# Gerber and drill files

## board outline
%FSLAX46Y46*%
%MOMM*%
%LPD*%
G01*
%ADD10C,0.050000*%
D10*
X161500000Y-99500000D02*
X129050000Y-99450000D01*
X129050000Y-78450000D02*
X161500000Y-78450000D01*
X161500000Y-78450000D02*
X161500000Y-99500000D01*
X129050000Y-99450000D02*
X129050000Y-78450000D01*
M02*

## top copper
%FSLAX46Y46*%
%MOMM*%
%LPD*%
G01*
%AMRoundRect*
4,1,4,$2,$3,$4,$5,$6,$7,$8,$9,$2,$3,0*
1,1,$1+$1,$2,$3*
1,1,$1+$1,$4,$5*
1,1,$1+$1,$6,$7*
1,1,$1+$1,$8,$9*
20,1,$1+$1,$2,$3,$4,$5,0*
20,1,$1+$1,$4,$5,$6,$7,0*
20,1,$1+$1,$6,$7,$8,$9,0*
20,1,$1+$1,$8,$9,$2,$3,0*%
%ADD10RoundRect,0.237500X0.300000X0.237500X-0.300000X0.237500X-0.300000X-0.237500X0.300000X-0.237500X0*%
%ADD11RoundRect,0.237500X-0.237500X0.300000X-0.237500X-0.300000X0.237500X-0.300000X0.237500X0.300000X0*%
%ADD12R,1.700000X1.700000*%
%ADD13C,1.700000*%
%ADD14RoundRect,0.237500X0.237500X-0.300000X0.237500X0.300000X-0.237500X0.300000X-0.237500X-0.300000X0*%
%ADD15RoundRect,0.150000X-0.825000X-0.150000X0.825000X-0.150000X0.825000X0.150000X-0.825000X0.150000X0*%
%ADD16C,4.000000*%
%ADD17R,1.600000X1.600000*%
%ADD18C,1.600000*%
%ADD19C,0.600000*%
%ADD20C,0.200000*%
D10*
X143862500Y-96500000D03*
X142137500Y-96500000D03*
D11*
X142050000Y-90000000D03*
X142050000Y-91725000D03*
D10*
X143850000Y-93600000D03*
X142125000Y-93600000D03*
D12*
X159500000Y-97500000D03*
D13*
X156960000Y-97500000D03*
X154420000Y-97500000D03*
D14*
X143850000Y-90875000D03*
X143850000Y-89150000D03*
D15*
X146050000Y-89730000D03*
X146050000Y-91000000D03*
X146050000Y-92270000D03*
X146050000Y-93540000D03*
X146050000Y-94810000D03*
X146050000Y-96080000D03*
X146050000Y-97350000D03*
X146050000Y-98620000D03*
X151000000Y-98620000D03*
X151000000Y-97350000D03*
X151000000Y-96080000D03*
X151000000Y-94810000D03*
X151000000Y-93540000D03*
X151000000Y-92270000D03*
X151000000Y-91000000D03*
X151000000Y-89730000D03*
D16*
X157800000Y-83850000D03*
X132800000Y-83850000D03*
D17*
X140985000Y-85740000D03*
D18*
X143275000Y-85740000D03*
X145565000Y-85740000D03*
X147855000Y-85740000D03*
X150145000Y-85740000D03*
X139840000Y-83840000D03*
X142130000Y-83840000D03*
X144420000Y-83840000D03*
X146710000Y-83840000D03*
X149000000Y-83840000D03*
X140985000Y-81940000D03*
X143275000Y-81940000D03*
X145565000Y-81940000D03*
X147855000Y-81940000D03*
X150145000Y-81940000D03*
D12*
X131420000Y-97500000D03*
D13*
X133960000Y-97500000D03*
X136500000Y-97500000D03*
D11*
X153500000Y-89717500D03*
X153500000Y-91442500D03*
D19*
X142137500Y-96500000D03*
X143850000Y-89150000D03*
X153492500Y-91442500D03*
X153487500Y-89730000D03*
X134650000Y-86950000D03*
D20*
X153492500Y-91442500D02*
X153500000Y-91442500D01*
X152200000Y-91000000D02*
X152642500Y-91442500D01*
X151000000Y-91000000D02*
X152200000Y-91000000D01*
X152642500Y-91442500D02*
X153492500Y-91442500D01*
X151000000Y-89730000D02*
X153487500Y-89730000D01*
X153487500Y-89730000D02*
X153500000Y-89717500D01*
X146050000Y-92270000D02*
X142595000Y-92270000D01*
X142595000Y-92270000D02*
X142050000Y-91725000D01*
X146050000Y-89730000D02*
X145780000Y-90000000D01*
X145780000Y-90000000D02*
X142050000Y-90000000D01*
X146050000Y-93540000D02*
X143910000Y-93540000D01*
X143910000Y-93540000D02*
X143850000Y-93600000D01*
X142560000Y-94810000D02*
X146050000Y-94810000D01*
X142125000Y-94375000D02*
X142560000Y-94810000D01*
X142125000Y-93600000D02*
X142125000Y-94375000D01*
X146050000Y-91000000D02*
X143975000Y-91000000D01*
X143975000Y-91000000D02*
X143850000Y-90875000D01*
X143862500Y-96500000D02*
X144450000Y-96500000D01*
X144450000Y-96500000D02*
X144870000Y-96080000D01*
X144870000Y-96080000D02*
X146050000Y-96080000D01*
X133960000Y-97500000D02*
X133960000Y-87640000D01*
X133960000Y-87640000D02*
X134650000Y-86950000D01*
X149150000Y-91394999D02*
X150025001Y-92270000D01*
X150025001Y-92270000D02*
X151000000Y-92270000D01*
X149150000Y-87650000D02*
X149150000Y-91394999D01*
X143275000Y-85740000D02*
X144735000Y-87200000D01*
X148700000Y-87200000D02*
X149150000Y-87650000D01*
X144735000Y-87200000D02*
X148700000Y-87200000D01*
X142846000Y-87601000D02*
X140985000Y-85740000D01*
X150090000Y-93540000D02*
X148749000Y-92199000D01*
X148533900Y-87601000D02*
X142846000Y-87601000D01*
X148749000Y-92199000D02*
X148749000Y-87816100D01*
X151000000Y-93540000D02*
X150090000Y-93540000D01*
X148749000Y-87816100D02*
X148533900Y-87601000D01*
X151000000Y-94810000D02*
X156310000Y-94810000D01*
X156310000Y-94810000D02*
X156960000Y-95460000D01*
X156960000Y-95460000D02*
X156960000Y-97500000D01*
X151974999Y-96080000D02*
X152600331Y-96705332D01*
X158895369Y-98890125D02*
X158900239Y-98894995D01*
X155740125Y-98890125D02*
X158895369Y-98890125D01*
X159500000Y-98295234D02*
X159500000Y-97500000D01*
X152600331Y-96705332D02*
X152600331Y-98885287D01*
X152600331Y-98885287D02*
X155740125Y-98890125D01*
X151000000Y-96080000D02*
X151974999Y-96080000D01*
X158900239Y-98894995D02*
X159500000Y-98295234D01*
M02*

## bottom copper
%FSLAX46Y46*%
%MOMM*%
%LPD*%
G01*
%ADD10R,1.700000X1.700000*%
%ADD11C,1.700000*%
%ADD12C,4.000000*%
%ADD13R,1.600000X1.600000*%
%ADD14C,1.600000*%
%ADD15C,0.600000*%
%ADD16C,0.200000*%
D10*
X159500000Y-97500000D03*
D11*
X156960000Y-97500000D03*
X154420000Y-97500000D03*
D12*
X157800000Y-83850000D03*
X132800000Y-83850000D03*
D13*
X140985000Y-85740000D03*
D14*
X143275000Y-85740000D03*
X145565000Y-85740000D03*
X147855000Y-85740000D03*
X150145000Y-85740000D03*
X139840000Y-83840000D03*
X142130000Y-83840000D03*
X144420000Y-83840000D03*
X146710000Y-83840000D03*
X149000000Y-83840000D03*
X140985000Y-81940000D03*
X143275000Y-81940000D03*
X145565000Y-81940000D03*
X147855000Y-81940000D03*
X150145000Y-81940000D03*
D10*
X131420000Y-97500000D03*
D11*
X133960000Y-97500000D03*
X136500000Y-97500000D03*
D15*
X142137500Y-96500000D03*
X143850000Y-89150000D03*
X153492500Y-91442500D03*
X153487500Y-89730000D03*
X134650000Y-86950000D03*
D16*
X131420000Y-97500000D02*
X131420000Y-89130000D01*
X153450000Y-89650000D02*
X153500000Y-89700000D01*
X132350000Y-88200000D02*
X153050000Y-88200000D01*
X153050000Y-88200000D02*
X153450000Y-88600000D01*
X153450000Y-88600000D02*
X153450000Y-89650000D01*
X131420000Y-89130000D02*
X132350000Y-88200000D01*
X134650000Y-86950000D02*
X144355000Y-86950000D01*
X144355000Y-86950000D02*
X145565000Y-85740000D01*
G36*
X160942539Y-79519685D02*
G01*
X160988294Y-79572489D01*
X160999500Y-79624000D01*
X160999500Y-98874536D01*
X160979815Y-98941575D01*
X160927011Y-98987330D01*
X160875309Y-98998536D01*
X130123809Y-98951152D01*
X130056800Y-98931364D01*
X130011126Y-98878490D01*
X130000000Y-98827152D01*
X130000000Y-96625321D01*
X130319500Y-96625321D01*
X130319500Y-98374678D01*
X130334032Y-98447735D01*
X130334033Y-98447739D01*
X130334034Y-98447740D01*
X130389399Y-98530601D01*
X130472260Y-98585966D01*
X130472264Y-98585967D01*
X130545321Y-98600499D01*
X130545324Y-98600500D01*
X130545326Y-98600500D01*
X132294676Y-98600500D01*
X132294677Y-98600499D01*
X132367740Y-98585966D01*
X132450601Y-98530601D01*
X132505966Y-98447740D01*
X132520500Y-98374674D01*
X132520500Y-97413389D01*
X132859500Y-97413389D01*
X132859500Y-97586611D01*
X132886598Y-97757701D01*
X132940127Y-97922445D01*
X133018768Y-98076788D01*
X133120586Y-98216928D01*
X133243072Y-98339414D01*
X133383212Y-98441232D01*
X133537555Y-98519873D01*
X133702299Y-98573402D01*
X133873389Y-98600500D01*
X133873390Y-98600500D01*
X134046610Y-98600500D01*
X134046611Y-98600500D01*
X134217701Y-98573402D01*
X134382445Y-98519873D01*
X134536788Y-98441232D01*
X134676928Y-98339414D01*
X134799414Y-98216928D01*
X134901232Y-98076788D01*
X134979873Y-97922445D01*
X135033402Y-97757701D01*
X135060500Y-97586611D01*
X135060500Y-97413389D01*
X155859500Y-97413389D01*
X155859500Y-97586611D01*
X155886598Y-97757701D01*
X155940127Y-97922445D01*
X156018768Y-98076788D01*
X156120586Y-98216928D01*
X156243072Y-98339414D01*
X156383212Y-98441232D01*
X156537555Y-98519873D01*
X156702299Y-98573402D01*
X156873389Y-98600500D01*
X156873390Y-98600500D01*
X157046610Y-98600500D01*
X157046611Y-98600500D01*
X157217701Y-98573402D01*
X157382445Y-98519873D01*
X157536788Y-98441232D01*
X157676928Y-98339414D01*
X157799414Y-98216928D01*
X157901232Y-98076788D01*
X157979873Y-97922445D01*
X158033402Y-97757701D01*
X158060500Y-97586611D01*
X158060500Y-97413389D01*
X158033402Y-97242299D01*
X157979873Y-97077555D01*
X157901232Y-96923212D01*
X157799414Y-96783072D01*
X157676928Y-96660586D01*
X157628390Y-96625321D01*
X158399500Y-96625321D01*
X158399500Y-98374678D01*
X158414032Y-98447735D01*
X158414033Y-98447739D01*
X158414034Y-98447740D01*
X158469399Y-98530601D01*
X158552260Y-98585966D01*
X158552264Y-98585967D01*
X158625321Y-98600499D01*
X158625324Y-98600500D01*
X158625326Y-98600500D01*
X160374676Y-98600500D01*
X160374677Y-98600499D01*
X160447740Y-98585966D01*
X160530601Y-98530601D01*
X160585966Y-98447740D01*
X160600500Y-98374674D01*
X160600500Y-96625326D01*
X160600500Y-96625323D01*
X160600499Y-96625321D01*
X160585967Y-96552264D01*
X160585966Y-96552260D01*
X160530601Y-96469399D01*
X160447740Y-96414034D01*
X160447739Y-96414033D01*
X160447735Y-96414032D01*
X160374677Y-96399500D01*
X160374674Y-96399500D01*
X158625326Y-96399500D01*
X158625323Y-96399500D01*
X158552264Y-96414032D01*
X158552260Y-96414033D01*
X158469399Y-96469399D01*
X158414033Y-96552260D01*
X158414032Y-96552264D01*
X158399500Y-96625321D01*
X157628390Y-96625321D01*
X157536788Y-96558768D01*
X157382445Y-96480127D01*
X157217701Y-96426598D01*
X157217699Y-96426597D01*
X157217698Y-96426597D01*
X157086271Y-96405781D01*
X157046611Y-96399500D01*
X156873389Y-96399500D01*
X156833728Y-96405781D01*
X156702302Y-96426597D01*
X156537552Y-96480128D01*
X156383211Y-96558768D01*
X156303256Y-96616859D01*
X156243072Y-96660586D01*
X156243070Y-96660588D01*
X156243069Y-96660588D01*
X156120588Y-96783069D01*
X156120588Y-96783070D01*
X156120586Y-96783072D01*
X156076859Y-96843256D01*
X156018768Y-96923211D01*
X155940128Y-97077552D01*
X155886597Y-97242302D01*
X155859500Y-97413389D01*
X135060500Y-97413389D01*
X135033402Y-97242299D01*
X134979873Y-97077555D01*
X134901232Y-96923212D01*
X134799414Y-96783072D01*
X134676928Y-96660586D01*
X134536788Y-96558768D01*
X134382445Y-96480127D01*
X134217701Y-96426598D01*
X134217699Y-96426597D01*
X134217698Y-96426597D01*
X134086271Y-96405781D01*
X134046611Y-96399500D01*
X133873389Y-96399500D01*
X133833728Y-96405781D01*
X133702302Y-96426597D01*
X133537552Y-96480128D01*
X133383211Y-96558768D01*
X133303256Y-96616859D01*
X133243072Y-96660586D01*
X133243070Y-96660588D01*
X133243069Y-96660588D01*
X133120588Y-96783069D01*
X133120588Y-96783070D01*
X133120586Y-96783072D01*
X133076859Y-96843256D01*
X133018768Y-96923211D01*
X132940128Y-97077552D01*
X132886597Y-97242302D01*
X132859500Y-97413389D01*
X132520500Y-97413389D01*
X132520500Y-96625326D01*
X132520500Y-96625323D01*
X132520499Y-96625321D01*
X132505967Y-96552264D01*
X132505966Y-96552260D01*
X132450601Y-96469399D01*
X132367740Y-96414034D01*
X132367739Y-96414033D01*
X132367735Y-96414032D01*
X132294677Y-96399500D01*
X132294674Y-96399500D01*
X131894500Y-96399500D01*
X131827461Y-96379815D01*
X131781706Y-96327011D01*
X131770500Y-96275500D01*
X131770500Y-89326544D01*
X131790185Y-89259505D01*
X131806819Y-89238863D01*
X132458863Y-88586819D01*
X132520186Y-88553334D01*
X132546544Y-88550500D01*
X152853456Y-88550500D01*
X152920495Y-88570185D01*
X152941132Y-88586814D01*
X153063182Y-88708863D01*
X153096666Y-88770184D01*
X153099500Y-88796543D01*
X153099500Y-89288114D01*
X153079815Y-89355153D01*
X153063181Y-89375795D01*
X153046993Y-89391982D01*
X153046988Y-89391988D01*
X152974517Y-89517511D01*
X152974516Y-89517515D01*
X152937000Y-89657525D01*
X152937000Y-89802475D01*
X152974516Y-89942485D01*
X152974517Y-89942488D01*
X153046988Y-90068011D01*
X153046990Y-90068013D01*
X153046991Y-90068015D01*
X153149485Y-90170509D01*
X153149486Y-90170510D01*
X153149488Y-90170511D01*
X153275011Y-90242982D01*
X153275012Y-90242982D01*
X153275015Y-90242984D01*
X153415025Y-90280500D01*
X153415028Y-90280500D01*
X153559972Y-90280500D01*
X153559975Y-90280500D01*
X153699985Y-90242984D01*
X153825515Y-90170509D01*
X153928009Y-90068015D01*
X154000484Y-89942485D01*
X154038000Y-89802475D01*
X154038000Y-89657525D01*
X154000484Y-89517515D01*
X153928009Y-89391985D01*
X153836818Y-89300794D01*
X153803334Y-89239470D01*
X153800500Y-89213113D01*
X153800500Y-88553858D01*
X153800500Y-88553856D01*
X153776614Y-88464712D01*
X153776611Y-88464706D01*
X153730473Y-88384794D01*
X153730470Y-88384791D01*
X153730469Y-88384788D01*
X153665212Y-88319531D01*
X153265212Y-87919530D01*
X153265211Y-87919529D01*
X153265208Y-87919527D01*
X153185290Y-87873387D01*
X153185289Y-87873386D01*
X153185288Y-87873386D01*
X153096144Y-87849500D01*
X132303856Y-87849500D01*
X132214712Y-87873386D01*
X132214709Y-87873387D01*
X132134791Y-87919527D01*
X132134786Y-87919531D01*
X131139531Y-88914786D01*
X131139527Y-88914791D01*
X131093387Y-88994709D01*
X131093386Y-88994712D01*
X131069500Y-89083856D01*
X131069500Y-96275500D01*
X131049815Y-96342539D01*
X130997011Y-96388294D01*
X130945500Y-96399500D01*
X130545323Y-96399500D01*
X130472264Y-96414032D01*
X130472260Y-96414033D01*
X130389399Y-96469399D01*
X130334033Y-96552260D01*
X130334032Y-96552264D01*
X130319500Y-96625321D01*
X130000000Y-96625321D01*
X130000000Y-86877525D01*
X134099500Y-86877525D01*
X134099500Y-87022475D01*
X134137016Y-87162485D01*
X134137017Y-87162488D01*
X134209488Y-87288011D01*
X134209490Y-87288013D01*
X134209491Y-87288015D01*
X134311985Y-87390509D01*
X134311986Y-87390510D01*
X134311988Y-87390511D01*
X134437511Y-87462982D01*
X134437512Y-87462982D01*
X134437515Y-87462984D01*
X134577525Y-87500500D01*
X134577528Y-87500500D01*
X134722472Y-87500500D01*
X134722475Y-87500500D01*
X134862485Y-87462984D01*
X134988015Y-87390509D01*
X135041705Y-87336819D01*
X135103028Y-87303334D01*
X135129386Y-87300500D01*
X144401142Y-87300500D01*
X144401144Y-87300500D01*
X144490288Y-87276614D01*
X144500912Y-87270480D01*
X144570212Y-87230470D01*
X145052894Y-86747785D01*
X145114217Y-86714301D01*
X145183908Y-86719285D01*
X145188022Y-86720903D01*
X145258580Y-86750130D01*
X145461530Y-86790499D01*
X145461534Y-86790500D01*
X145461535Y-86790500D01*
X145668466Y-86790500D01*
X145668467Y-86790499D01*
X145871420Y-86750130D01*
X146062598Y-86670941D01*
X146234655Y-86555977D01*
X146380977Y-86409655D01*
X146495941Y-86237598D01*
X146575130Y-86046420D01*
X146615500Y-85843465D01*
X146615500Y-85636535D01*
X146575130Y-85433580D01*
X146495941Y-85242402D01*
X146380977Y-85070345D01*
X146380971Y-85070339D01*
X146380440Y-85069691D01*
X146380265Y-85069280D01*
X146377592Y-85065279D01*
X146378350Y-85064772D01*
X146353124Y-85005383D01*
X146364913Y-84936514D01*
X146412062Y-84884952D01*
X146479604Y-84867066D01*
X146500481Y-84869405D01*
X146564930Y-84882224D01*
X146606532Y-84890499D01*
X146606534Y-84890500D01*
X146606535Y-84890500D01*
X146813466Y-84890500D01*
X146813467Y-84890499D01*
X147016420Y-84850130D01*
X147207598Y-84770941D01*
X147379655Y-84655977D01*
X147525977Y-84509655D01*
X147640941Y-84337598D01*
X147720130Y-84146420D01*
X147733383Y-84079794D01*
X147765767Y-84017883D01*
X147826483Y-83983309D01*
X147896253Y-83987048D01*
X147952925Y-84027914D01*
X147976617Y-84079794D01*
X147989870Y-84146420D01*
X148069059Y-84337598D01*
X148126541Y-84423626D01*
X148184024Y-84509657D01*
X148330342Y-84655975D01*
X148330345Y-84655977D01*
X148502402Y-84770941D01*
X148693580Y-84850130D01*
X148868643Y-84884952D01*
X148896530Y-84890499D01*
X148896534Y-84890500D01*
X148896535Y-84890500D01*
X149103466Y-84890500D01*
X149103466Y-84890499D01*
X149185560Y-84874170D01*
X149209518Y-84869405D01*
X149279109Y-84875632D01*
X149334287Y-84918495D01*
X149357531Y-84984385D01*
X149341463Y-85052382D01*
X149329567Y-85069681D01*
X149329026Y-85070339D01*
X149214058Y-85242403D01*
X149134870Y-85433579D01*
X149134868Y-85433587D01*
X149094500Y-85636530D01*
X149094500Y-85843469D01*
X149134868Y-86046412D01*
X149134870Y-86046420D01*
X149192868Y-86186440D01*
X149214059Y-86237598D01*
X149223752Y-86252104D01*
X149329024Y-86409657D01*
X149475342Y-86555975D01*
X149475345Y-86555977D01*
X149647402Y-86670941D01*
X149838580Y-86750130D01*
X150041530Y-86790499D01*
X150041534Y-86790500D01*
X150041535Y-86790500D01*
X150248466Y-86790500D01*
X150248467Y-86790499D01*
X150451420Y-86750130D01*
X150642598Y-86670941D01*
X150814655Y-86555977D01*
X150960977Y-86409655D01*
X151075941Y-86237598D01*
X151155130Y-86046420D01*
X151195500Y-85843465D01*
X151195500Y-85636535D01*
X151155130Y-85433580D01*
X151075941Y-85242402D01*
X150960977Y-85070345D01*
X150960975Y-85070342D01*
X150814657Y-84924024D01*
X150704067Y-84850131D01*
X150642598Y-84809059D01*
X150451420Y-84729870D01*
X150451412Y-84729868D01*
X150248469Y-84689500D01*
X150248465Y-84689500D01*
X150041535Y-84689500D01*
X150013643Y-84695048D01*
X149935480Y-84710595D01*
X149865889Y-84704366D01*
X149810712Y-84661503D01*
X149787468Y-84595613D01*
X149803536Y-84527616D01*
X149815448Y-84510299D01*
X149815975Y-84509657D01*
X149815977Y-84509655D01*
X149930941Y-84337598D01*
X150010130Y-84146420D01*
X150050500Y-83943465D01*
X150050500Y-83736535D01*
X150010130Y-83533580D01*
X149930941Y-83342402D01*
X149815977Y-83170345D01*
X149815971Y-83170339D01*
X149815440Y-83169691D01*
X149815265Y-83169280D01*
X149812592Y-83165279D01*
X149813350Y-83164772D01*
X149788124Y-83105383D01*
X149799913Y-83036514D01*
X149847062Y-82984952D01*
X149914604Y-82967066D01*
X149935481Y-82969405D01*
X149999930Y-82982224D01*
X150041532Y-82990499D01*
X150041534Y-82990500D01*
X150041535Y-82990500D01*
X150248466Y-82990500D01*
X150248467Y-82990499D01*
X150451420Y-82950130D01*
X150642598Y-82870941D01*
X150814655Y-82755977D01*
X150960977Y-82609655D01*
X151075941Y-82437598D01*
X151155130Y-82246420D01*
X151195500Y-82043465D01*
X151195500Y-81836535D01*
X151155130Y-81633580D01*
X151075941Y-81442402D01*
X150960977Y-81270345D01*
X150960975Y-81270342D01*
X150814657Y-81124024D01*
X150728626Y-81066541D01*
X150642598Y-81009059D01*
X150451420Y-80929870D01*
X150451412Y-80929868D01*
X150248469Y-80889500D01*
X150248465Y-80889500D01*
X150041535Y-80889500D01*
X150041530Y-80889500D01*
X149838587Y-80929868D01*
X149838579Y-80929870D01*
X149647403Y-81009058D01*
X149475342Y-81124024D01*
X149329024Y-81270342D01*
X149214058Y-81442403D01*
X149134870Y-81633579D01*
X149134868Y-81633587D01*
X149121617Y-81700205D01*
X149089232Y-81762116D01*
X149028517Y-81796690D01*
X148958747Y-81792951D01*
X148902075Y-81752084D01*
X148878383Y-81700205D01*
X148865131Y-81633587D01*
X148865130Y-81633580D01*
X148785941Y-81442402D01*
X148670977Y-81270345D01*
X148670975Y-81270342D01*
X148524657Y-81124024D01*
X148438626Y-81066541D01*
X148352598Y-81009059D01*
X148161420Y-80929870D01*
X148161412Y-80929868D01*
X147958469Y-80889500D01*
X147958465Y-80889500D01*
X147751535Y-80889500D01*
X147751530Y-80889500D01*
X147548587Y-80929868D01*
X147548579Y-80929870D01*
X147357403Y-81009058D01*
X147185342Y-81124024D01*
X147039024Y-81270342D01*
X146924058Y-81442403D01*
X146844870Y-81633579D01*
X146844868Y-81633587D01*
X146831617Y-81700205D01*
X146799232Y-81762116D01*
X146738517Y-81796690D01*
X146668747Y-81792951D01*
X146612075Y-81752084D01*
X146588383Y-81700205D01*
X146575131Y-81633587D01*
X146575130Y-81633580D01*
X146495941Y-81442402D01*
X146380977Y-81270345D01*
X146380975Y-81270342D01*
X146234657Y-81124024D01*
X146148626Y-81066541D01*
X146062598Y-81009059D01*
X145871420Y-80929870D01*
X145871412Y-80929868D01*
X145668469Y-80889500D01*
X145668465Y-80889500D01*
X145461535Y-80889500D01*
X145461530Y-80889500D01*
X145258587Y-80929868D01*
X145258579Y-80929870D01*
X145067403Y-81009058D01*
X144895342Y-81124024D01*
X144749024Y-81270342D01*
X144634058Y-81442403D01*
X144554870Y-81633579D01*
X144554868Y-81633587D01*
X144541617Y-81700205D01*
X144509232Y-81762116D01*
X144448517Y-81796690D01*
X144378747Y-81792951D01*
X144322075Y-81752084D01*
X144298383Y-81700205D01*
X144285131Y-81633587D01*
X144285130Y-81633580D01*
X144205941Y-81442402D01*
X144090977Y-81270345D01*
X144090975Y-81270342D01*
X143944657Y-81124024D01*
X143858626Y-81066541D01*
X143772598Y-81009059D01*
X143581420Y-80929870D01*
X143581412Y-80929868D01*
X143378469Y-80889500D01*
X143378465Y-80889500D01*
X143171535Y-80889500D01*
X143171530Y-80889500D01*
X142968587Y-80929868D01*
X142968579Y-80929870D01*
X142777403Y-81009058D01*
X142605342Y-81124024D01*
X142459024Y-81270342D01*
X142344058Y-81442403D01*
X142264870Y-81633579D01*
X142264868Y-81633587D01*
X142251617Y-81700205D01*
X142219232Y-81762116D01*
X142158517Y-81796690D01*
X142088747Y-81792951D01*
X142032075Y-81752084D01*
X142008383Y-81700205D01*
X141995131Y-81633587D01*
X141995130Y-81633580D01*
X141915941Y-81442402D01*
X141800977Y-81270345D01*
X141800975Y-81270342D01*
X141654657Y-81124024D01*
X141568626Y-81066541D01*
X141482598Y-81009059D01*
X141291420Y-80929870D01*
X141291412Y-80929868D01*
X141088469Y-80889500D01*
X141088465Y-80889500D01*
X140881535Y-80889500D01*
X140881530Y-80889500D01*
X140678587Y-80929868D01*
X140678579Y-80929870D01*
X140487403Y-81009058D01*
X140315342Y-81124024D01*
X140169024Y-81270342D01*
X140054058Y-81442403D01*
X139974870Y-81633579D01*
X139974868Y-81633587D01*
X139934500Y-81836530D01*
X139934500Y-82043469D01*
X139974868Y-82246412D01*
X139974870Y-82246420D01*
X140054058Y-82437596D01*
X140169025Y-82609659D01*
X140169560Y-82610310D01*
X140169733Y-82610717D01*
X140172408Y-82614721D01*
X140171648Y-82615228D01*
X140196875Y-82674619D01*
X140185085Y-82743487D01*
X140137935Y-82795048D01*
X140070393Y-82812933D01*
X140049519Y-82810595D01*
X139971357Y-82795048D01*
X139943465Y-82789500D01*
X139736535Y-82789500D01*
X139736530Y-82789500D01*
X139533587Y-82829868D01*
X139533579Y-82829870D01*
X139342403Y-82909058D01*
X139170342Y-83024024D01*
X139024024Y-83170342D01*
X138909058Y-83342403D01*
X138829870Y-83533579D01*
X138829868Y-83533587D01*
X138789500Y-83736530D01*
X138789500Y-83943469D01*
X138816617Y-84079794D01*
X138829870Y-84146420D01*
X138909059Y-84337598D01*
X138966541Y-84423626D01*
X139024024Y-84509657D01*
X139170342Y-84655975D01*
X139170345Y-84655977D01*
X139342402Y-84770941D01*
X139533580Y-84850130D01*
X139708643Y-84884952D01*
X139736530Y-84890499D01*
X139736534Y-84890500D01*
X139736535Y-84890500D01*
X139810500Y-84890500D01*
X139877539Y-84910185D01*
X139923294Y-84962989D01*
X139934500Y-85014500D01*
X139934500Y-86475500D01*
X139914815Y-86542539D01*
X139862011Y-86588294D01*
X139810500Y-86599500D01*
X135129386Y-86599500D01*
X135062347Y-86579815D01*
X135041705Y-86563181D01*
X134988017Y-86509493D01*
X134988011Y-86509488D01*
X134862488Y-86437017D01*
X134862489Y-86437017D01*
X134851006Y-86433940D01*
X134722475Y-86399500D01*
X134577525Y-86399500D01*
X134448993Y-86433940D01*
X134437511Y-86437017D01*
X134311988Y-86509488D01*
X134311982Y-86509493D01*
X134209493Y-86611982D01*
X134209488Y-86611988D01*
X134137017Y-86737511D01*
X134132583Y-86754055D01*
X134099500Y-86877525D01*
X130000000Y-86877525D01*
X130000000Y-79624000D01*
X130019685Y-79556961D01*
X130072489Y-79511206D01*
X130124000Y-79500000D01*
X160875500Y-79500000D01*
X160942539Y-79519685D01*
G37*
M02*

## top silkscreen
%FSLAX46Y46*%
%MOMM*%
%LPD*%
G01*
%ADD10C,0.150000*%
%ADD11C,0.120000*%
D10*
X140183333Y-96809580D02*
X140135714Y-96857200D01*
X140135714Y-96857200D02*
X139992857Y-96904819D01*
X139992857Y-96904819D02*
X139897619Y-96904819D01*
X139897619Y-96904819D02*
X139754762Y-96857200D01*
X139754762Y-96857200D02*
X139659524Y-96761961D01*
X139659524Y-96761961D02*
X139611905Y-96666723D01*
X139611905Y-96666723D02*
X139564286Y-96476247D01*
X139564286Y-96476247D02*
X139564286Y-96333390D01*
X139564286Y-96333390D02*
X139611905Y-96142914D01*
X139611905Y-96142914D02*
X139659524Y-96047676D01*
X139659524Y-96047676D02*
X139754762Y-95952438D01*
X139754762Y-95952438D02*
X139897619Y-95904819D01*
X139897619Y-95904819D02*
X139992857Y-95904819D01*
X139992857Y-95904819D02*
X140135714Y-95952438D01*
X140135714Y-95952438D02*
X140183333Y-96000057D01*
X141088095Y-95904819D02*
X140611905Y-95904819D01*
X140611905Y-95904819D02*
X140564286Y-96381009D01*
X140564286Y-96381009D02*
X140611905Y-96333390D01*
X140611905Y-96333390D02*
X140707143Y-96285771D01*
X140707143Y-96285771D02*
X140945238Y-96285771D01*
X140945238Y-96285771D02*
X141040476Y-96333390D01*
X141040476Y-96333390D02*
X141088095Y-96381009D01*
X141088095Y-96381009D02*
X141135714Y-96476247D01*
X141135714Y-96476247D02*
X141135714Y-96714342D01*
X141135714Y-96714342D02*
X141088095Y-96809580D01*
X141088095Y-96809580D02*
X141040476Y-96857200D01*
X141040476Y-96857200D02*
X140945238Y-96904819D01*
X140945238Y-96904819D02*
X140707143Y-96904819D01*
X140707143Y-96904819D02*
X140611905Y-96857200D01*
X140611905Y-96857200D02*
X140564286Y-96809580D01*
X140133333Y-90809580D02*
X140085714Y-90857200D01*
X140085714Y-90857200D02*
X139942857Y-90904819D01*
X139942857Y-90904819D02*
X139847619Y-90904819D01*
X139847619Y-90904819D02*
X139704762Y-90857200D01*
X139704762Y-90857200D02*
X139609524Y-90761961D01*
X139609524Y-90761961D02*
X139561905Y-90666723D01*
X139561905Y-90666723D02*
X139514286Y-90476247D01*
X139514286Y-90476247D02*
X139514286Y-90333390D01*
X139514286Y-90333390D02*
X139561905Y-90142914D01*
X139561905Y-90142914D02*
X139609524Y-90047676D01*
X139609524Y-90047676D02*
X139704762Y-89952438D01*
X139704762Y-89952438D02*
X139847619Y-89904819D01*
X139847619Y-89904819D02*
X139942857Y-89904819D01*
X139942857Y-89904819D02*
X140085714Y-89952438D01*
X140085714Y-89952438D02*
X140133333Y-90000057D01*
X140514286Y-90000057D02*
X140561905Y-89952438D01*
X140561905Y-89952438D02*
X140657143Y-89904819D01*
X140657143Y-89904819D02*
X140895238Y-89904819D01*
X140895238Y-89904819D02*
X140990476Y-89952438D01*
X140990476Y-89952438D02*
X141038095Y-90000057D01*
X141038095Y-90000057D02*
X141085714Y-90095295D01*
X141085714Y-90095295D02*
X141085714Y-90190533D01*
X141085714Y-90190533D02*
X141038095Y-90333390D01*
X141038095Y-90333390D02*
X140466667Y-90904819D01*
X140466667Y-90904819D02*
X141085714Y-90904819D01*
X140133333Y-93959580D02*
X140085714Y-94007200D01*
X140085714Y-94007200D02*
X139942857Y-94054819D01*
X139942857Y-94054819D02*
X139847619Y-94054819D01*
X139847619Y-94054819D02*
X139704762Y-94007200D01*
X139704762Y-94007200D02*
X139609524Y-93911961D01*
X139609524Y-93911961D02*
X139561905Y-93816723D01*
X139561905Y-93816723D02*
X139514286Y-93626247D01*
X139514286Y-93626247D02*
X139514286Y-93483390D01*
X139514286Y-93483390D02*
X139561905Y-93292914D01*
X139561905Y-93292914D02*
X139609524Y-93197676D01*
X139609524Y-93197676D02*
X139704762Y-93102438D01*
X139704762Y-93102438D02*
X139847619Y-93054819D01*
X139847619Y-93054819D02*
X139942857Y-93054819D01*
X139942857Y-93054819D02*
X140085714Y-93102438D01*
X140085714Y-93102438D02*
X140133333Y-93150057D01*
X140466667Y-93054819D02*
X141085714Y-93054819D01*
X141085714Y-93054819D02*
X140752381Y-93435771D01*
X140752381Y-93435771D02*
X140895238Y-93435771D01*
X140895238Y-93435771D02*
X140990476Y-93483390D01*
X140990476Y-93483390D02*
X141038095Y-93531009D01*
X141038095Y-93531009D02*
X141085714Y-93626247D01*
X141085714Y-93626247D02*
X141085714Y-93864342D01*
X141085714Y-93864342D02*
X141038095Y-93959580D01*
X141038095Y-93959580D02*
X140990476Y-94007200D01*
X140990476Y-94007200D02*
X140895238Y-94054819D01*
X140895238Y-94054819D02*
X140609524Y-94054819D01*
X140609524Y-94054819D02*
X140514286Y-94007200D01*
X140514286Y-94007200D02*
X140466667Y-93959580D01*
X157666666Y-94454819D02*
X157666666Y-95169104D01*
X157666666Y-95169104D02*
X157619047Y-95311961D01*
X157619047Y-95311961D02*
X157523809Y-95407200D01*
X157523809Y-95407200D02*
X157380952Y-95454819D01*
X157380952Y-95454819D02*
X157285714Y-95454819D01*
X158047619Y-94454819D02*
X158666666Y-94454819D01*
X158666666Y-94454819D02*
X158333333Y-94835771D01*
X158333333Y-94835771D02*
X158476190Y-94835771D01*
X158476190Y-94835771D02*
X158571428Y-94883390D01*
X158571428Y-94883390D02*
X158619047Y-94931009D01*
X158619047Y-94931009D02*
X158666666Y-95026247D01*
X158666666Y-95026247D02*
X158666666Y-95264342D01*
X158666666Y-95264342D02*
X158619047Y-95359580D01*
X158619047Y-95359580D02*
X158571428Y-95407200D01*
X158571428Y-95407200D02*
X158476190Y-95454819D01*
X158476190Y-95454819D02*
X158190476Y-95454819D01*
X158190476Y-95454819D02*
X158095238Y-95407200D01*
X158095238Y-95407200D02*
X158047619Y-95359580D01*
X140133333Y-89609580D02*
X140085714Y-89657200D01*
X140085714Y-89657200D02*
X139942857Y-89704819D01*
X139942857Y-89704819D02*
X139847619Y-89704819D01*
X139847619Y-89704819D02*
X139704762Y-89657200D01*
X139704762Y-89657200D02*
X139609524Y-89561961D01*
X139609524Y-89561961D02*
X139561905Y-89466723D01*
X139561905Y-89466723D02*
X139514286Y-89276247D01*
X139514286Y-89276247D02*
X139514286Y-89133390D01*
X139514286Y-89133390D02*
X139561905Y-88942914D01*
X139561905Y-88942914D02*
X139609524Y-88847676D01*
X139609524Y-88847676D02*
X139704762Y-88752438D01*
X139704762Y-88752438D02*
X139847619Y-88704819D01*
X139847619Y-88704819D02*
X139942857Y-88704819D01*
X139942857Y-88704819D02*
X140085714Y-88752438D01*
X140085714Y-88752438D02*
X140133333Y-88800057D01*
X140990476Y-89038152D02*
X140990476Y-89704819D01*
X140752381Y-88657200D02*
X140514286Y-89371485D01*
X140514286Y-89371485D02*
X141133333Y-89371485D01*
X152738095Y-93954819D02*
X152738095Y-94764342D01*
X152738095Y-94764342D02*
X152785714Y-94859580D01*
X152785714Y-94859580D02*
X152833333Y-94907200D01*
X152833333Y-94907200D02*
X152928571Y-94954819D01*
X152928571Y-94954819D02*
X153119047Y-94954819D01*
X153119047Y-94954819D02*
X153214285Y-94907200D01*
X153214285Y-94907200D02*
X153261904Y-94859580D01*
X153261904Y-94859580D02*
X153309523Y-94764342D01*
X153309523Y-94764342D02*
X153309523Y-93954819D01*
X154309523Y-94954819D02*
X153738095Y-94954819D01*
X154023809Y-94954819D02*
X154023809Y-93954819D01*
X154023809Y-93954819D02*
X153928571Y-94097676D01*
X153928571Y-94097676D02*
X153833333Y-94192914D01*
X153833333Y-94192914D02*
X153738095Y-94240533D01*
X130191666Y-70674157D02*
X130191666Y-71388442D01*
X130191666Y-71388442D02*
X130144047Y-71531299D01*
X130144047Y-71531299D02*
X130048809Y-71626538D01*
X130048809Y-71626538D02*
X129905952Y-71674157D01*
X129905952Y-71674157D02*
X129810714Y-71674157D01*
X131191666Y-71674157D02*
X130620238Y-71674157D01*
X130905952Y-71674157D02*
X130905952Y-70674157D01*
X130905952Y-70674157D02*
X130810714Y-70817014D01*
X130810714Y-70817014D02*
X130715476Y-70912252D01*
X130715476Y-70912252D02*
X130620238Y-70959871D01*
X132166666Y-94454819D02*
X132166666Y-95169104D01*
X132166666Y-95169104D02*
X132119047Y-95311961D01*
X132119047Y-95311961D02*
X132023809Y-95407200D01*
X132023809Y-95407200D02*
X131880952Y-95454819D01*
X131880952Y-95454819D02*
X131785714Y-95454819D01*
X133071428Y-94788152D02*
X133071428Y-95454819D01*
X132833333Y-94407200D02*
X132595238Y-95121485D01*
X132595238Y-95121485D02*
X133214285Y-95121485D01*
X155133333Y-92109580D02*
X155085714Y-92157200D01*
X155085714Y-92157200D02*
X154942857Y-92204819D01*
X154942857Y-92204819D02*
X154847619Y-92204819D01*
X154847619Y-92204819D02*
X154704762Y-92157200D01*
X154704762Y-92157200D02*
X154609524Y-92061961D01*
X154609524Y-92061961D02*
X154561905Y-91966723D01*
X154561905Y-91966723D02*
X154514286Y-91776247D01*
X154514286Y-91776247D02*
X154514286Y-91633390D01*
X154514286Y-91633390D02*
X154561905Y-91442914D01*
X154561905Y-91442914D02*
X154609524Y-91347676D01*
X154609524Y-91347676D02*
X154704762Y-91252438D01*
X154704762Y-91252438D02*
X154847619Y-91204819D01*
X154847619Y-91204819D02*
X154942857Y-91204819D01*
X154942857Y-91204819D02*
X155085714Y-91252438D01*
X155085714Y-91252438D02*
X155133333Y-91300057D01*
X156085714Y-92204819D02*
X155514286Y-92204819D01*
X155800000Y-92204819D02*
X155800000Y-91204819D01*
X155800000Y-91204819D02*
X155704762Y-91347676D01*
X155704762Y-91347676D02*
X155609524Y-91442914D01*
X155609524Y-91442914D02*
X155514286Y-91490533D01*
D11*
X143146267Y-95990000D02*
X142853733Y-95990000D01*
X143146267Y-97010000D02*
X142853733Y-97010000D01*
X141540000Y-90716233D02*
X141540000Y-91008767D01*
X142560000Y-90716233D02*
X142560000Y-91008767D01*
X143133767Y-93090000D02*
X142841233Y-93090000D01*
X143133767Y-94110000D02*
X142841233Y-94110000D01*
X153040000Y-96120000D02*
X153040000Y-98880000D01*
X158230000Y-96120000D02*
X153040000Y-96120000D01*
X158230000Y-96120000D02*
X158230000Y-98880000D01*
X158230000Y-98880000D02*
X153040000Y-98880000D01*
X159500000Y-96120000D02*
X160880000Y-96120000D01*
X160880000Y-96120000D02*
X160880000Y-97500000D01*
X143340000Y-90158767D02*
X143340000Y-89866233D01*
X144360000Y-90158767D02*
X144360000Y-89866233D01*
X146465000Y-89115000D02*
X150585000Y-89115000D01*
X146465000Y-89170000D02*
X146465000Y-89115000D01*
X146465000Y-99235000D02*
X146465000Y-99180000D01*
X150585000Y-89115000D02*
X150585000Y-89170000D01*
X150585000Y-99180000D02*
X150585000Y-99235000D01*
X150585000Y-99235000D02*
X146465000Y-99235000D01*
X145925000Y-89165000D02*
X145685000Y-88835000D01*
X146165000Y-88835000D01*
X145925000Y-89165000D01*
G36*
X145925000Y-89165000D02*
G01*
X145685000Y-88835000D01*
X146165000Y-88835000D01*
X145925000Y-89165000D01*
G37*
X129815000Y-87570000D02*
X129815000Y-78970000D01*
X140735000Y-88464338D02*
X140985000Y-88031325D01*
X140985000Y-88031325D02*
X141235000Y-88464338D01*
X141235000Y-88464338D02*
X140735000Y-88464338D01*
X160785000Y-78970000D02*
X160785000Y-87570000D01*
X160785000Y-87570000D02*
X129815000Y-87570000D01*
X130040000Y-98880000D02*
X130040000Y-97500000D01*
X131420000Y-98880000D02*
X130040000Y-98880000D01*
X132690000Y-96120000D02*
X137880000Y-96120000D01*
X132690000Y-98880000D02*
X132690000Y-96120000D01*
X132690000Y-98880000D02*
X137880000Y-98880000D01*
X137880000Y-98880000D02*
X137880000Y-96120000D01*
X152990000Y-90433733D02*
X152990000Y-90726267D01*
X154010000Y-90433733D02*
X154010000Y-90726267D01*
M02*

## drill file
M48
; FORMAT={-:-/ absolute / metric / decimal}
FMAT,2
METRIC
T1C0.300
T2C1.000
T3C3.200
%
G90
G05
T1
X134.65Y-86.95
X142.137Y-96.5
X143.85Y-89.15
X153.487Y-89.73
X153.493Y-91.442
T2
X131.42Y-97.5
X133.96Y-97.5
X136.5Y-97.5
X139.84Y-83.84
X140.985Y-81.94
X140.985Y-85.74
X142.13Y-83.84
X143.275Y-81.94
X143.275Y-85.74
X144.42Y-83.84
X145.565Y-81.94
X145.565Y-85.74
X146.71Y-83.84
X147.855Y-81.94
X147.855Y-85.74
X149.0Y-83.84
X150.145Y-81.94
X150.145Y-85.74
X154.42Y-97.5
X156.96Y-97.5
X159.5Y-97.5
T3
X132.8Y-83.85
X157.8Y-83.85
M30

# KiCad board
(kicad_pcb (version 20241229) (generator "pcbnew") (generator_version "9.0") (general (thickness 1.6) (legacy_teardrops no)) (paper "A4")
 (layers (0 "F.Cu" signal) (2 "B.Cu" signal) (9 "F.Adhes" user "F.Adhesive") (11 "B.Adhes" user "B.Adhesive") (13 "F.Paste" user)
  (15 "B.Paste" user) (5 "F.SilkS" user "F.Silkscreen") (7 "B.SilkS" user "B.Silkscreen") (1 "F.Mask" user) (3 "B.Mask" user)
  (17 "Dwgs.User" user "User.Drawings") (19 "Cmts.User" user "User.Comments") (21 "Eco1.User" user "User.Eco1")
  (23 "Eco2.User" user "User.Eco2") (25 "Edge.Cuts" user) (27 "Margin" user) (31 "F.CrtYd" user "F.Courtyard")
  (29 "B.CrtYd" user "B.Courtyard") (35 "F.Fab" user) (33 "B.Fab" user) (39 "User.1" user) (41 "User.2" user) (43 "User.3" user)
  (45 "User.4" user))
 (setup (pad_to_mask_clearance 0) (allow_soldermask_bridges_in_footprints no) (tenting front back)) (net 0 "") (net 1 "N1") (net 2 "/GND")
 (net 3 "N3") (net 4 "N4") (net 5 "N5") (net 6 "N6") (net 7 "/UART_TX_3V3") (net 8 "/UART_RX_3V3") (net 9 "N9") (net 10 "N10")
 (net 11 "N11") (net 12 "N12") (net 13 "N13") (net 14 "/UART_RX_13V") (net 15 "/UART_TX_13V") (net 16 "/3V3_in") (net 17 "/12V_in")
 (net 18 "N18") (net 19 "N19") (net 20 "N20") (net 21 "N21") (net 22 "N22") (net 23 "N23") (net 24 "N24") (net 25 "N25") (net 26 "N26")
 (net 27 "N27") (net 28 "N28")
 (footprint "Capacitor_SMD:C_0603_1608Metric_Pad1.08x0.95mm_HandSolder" (layer "F.Cu") (at 143 96.5 180)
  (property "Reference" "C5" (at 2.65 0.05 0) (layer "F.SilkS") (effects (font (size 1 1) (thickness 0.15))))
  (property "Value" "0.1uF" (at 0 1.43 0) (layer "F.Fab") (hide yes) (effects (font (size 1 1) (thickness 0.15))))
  (fp_line (start -0.146267 0.51) (end 0.146267 0.51) (stroke (width 0.12) (type solid)) (layer "F.SilkS"))
  (fp_line (start -0.146267 -0.51) (end 0.146267 -0.51) (stroke (width 0.12) (type solid)) (layer "F.SilkS"))
  (pad "1" smd roundrect (at -0.8625 0 180) (size 1.075 0.95) (layers "F.Cu" "F.Mask" "F.Paste") (roundrect_rratio 0.25) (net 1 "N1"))
  (pad "2" smd roundrect (at 0.8625 0 180) (size 1.075 0.95) (layers "F.Cu" "F.Mask" "F.Paste") (roundrect_rratio 0.25) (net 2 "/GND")))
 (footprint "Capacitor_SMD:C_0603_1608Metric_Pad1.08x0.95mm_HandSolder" (layer "F.Cu") (at 142.05 90.8625 -90)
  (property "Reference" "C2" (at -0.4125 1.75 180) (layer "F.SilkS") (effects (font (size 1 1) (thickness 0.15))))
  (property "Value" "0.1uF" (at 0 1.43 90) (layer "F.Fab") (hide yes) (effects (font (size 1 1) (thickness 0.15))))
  (fp_line (start -0.146267 0.51) (end 0.146267 0.51) (stroke (width 0.12) (type solid)) (layer "F.SilkS"))
  (fp_line (start -0.146267 -0.51) (end 0.146267 -0.51) (stroke (width 0.12) (type solid)) (layer "F.SilkS"))
  (pad "1" smd roundrect (at -0.8625 0 270) (size 1.075 0.95) (layers "F.Cu" "F.Mask" "F.Paste") (roundrect_rratio 0.25) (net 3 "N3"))
  (pad "2" smd roundrect (at 0.8625 0 270) (size 1.075 0.95) (layers "F.Cu" "F.Mask" "F.Paste") (roundrect_rratio 0.25) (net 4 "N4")))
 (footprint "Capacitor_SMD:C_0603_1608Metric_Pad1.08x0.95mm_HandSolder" (layer "F.Cu") (at 142.9875 93.6 180)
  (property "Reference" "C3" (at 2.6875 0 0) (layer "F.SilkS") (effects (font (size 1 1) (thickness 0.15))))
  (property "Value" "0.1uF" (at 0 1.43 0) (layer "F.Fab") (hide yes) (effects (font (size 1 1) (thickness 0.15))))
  (fp_line (start -0.146267 0.51) (end 0.146267 0.51) (stroke (width 0.12) (type solid)) (layer "F.SilkS"))
  (fp_line (start -0.146267 -0.51) (end 0.146267 -0.51) (stroke (width 0.12) (type solid)) (layer "F.SilkS"))
  (pad "1" smd roundrect (at -0.8625 0 180) (size 1.075 0.95) (layers "F.Cu" "F.Mask" "F.Paste") (roundrect_rratio 0.25) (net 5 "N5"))
  (pad "2" smd roundrect (at 0.8625 0 180) (size 1.075 0.95) (layers "F.Cu" "F.Mask" "F.Paste") (roundrect_rratio 0.25) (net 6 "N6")))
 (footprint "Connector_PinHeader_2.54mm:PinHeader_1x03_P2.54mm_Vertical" (layer "F.Cu") (at 159.5 97.5 -90)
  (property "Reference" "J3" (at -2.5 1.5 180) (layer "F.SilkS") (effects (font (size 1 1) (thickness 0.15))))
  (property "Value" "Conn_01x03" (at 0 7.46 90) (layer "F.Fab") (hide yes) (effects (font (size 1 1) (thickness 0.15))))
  (fp_line (start -1.38 6.46) (end 1.38 6.46) (stroke (width 0.12) (type solid)) (layer "F.SilkS"))
  (fp_line (start -1.38 1.27) (end -1.38 6.46) (stroke (width 0.12) (type solid)) (layer "F.SilkS"))
  (fp_line (start -1.38 1.27) (end 1.38 1.27) (stroke (width 0.12) (type solid)) (layer "F.SilkS"))
  (fp_line (start 1.38 1.27) (end 1.38 6.46) (stroke (width 0.12) (type solid)) (layer "F.SilkS"))
  (fp_line (start -1.38 0) (end -1.38 -1.38) (stroke (width 0.12) (type solid)) (layer "F.SilkS"))
  (fp_line (start -1.38 -1.38) (end 0 -1.38) (stroke (width 0.12) (type solid)) (layer "F.SilkS"))
  (pad "1" thru_hole rect (at 0 0 270) (size 1.7 1.7) (drill 1) (layers "*.Cu" "*.Mask") (remove_unused_layers no) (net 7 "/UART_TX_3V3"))
  (pad "2" thru_hole circle (at 0 2.54 270) (size 1.7 1.7) (drill 1) (layers "*.Cu" "*.Mask") (remove_unused_layers no)
   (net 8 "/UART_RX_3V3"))
  (pad "3" thru_hole circle (at 0 5.08 270) (size 1.7 1.7) (drill 1) (layers "*.Cu" "*.Mask") (remove_unused_layers no) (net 2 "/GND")))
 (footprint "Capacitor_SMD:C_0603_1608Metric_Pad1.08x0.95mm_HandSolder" (layer "F.Cu") (at 143.85 90.0125 90)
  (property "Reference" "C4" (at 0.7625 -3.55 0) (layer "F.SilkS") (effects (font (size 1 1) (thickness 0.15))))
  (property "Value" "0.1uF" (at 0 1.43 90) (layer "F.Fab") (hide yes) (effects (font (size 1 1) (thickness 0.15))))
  (fp_line (start -0.146267 -0.51) (end 0.146267 -0.51) (stroke (width 0.12) (type solid)) (layer "F.SilkS"))
  (fp_line (start -0.146267 0.51) (end 0.146267 0.51) (stroke (width 0.12) (type solid)) (layer "F.SilkS"))
  (pad "1" smd roundrect (at -0.8625 0 90) (size 1.075 0.95) (layers "F.Cu" "F.Mask" "F.Paste") (roundrect_rratio 0.25) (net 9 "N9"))
  (pad "2" smd roundrect (at 0.8625 0 90) (size 1.075 0.95) (layers "F.Cu" "F.Mask" "F.Paste") (roundrect_rratio 0.25) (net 2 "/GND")))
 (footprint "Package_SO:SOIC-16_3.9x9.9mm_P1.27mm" (layer "F.Cu") (at 148.525 94.175)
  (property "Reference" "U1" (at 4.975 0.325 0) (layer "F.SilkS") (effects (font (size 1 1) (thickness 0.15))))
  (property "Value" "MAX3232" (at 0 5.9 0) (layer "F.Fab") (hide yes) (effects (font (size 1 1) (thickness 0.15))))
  (fp_line (start -2.06 -5.06) (end 2.06 -5.06) (stroke (width 0.12) (type solid)) (layer "F.SilkS"))
  (fp_line (start -2.06 -5.005) (end -2.06 -5.06) (stroke (width 0.12) (type solid)) (layer "F.SilkS"))
  (fp_line (start -2.06 5.06) (end -2.06 5.005) (stroke (width 0.12) (type solid)) (layer "F.SilkS"))
  (fp_line (start 2.06 -5.06) (end 2.06 -5.005) (stroke (width 0.12) (type solid)) (layer "F.SilkS"))
  (fp_line (start 2.06 5.005) (end 2.06 5.06) (stroke (width 0.12) (type solid)) (layer "F.SilkS"))
  (fp_line (start 2.06 5.06) (end -2.06 5.06) (stroke (width 0.12) (type solid)) (layer "F.SilkS"))
  (fp_poly (pts (xy -2.6 -5.01) (xy -2.84 -5.34) (xy -2.36 -5.34)) (stroke (width 0.12) (type solid)) (fill yes) (layer "F.SilkS"))
  (pad "1" smd roundrect (at -2.475 -4.445) (size 1.95 0.6) (layers "F.Cu" "F.Mask" "F.Paste") (roundrect_rratio 0.25) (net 3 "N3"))
  (pad "2" smd roundrect (at -2.475 -3.175) (size 1.95 0.6) (layers "F.Cu" "F.Mask" "F.Paste") (roundrect_rratio 0.25) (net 9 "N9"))
  (pad "3" smd roundrect (at -2.475 -1.905) (size 1.95 0.6) (layers "F.Cu" "F.Mask" "F.Paste") (roundrect_rratio 0.25) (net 4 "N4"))
  (pad "4" smd roundrect (at -2.475 -0.635) (size 1.95 0.6) (layers "F.Cu" "F.Mask" "F.Paste") (roundrect_rratio 0.25) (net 5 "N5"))
  (pad "5" smd roundrect (at -2.475 0.635) (size 1.95 0.6) (layers "F.Cu" "F.Mask" "F.Paste") (roundrect_rratio 0.25) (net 6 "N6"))
  (pad "6" smd roundrect (at -2.475 1.905) (size 1.95 0.6) (layers "F.Cu" "F.Mask" "F.Paste") (roundrect_rratio 0.25) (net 1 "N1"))
  (pad "7" smd roundrect (at -2.475 3.175) (size 1.95 0.6) (layers "F.Cu" "F.Mask" "F.Paste") (roundrect_rratio 0.25) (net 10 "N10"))
  (pad "8" smd roundrect (at -2.475 4.445) (size 1.95 0.6) (layers "F.Cu" "F.Mask" "F.Paste") (roundrect_rratio 0.25) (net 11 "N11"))
  (pad "9" smd roundrect (at 2.475 4.445) (size 1.95 0.6) (layers "F.Cu" "F.Mask" "F.Paste") (roundrect_rratio 0.25) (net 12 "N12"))
  (pad "10" smd roundrect (at 2.475 3.175) (size 1.95 0.6) (layers "F.Cu" "F.Mask" "F.Paste") (roundrect_rratio 0.25) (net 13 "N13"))
  (pad "11" smd roundrect (at 2.475 1.905) (size 1.95 0.6) (layers "F.Cu" "F.Mask" "F.Paste") (roundrect_rratio 0.25) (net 7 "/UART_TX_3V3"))
  (pad "12" smd roundrect (at 2.475 0.635) (size 1.95 0.6) (layers "F.Cu" "F.Mask" "F.Paste") (roundrect_rratio 0.25) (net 8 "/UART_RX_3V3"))
  (pad "13" smd roundrect (at 2.475 -0.635) (size 1.95 0.6) (layers "F.Cu" "F.Mask" "F.Paste") (roundrect_rratio 0.25)
   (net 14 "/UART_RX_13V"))
  (pad "14" smd roundrect (at 2.475 -1.905) (size 1.95 0.6) (layers "F.Cu" "F.Mask" "F.Paste") (roundrect_rratio 0.25)
   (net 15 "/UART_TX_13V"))
  (pad "15" smd roundrect (at 2.475 -3.175) (size 1.95 0.6) (layers "F.Cu" "F.Mask" "F.Paste") (roundrect_rratio 0.25) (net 2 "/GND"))
  (pad "16" smd roundrect (at 2.475 -4.445) (size 1.95 0.6) (layers "F.Cu" "F.Mask" "F.Paste") (roundrect_rratio 0.25) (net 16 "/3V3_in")))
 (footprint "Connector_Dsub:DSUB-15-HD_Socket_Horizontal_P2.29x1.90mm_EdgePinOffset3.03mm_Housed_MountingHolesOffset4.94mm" (layer "F.Cu")
  (at 140.985 85.74 180)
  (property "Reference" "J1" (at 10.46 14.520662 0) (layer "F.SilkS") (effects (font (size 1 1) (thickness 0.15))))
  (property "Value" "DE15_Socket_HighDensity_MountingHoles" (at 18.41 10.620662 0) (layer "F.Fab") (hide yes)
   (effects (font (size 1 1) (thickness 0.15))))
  (fp_line (start 11.17 -1.83) (end 11.17 6.77) (stroke (width 0.12) (type solid)) (layer "F.SilkS"))
  (fp_line (start 0.25 -2.724338) (end 0 -2.291325) (stroke (width 0.12) (type solid)) (layer "F.SilkS"))
  (fp_line (start 0 -2.291325) (end -0.25 -2.724338) (stroke (width 0.12) (type solid)) (layer "F.SilkS"))
  (fp_line (start -0.25 -2.724338) (end 0.25 -2.724338) (stroke (width 0.12) (type solid)) (layer "F.SilkS"))
  (fp_line (start -19.8 6.77) (end -19.8 -1.83) (stroke (width 0.12) (type solid)) (layer "F.SilkS"))
  (fp_line (start -19.8 -1.83) (end 11.17 -1.83) (stroke (width 0.12) (type solid)) (layer "F.SilkS"))
  (pad "0" thru_hole circle (at -16.815 1.89 180) (size 4 4) (drill 3.2) (layers "*.Cu" "*.Mask") (remove_unused_layers no) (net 2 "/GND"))
  (pad "0" thru_hole circle (at 8.185 1.89 180) (size 4 4) (drill 3.2) (layers "*.Cu" "*.Mask") (remove_unused_layers no) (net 2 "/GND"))
  (pad "1" thru_hole rect (at 0 0 180) (size 1.6 1.6) (drill 1) (layers "*.Cu" "*.Mask") (remove_unused_layers no) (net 14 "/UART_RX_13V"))
  (pad "2" thru_hole circle (at -2.29 0 180) (size 1.6 1.6) (drill 1) (layers "*.Cu" "*.Mask") (remove_unused_layers no)
   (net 15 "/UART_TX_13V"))
  (pad "3" thru_hole circle (at -4.58 0 180) (size 1.6 1.6) (drill 1) (layers "*.Cu" "*.Mask") (remove_unused_layers no) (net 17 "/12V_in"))
  (pad "4" thru_hole circle (at -6.87 0 180) (size 1.6 1.6) (drill 1) (layers "*.Cu" "*.Mask") (remove_unused_layers no) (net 2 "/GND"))
  (pad "5" thru_hole circle (at -9.16 0 180) (size 1.6 1.6) (drill 1) (layers "*.Cu" "*.Mask") (remove_unused_layers no) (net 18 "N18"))
  (pad "6" thru_hole circle (at 1.145 1.9 180) (size 1.6 1.6) (drill 1) (layers "*.Cu" "*.Mask") (remove_unused_layers no) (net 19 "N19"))
  (pad "7" thru_hole circle (at -1.145 1.9 180) (size 1.6 1.6) (drill 1) (layers "*.Cu" "*.Mask") (remove_unused_layers no) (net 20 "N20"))
  (pad "8" thru_hole circle (at -3.435 1.9 180) (size 1.6 1.6) (drill 1) (layers "*.Cu" "*.Mask") (remove_unused_layers no) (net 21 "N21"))
  (pad "9" thru_hole circle (at -5.725 1.9 180) (size 1.6 1.6) (drill 1) (layers "*.Cu" "*.Mask") (remove_unused_layers no) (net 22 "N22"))
  (pad "10" thru_hole circle (at -8.015 1.9 180) (size 1.6 1.6) (drill 1) (layers "*.Cu" "*.Mask") (remove_unused_layers no) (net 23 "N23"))
  (pad "11" thru_hole circle (at 0 3.8 180) (size 1.6 1.6) (drill 1) (layers "*.Cu" "*.Mask") (remove_unused_layers no) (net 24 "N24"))
  (pad "12" thru_hole circle (at -2.29 3.8 180) (size 1.6 1.6) (drill 1) (layers "*.Cu" "*.Mask") (remove_unused_layers no) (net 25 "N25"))
  (pad "13" thru_hole circle (at -4.58 3.8 180) (size 1.6 1.6) (drill 1) (layers "*.Cu" "*.Mask") (remove_unused_layers no) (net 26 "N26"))
  (pad "14" thru_hole circle (at -6.87 3.8 180) (size 1.6 1.6) (drill 1) (layers "*.Cu" "*.Mask") (remove_unused_layers no) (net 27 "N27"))
  (pad "15" thru_hole circle (at -9.16 3.8 180) (size 1.6 1.6) (drill 1) (layers "*.Cu" "*.Mask") (remove_unused_layers no) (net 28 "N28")))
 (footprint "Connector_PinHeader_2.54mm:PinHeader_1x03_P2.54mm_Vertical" (layer "F.Cu") (at 131.42 97.5 90)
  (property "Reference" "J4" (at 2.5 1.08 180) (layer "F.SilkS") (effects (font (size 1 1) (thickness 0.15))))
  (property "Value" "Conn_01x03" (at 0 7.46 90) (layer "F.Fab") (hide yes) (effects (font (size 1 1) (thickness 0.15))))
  (fp_line (start -1.38 -1.38) (end 0 -1.38) (stroke (width 0.12) (type solid)) (layer "F.SilkS"))
  (fp_line (start -1.38 0) (end -1.38 -1.38) (stroke (width 0.12) (type solid)) (layer "F.SilkS"))
  (fp_line (start 1.38 1.27) (end 1.38 6.46) (stroke (width 0.12) (type solid)) (layer "F.SilkS"))
  (fp_line (start -1.38 1.27) (end 1.38 1.27) (stroke (width 0.12) (type solid)) (layer "F.SilkS"))
  (fp_line (start -1.38 1.27) (end -1.38 6.46) (stroke (width 0.12) (type solid)) (layer "F.SilkS"))
  (fp_line (start -1.38 6.46) (end 1.38 6.46) (stroke (width 0.12) (type solid)) (layer "F.SilkS"))
  (pad "1" thru_hole rect (at 0 0 90) (size 1.7 1.7) (drill 1) (layers "*.Cu" "*.Mask") (remove_unused_layers no) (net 16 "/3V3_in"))
  (pad "2" thru_hole circle (at 0 2.54 90) (size 1.7 1.7) (drill 1) (layers "*.Cu" "*.Mask") (remove_unused_layers no) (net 17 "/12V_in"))
  (pad "3" thru_hole circle (at 0 5.08 90) (size 1.7 1.7) (drill 1) (layers "*.Cu" "*.Mask") (remove_unused_layers no) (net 2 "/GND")))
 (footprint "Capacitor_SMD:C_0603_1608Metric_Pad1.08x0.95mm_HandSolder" (layer "F.Cu") (at 153.5 90.58 -90)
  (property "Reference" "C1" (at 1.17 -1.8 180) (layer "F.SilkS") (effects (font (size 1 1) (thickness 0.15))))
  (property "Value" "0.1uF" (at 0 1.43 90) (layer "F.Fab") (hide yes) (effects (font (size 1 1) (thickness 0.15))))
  (fp_line (start -0.146267 0.51) (end 0.146267 0.51) (stroke (width 0.12) (type solid)) (layer "F.SilkS"))
  (fp_line (start -0.146267 -0.51) (end 0.146267 -0.51) (stroke (width 0.12) (type solid)) (layer "F.SilkS"))
  (pad "1" smd roundrect (at -0.8625 0 270) (size 1.075 0.95) (layers "F.Cu" "F.Mask" "F.Paste") (roundrect_rratio 0.25) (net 16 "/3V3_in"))
  (pad "2" smd roundrect (at 0.8625 0 270) (size 1.075 0.95) (layers "F.Cu" "F.Mask" "F.Paste") (roundrect_rratio 0.25) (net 2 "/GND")))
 (gr_line (start 161.5 99.5) (end 129.05 99.45) (stroke (width 0.05) (type default)) (layer "Edge.Cuts"))
 (gr_line (start 129.05 78.45) (end 161.5 78.45) (stroke (width 0.05) (type default)) (layer "Edge.Cuts"))
 (gr_line (start 161.5 78.45) (end 161.5 99.5) (stroke (width 0.05) (type default)) (layer "Edge.Cuts"))
 (gr_line (start 129.05 99.45) (end 129.05 78.45) (stroke (width 0.05) (type default)) (layer "Edge.Cuts"))
 (segment (start 153.4925 91.4425) (end 153.5 91.4425) (width 0.2) (layer "F.Cu") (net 2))
 (segment (start 152.2 91) (end 152.6425 91.4425) (width 0.2) (layer "F.Cu") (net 2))
 (segment (start 151 91) (end 152.2 91) (width 0.2) (layer "F.Cu") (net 2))
 (segment (start 152.6425 91.4425) (end 153.4925 91.4425) (width 0.2) (layer "F.Cu") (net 2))
 (via (at 142.1375 96.5) (size 0.6) (drill 0.3) (layers "F.Cu" "B.Cu") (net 2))
 (via (at 143.85 89.15) (size 0.6) (drill 0.3) (layers "F.Cu" "B.Cu") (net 2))
 (via (at 153.4925 91.4425) (size 0.6) (drill 0.3) (layers "F.Cu" "B.Cu") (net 2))
 (segment (start 151 89.73) (end 153.4875 89.73) (width 0.2) (layer "F.Cu") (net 16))
 (segment (start 153.4875 89.73) (end 153.5 89.7175) (width 0.2) (layer "F.Cu") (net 16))
 (via (at 153.4875 89.73) (size 0.6) (drill 0.3) (layers "F.Cu" "B.Cu") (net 16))
 (segment (start 131.42 97.5) (end 131.42 89.13) (width 0.2) (layer "B.Cu") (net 16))
 (segment (start 153.45 89.65) (end 153.5 89.7) (width 0.2) (layer "B.Cu") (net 16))
 (segment (start 132.35 88.2) (end 153.05 88.2) (width 0.2) (layer "B.Cu") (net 16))
 (segment (start 153.05 88.2) (end 153.45 88.6) (width 0.2) (layer "B.Cu") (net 16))
 (segment (start 153.45 88.6) (end 153.45 89.65) (width 0.2) (layer "B.Cu") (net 16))
 (segment (start 131.42 89.13) (end 132.35 88.2) (width 0.2) (layer "B.Cu") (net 16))
 (segment (start 146.05 92.27) (end 142.595 92.27) (width 0.2) (layer "F.Cu") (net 4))
 (segment (start 142.595 92.27) (end 142.05 91.725) (width 0.2) (layer "F.Cu") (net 4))
 (segment (start 146.05 89.73) (end 145.78 90) (width 0.2) (layer "F.Cu") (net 3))
 (segment (start 145.78 90) (end 142.05 90) (width 0.2) (layer "F.Cu") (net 3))
 (segment (start 146.05 93.54) (end 143.91 93.54) (width 0.2) (layer "F.Cu") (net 5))
 (segment (start 143.91 93.54) (end 143.85 93.6) (width 0.2) (layer "F.Cu") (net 5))
 (segment (start 142.56 94.81) (end 146.05 94.81) (width 0.2) (layer "F.Cu") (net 6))
 (segment (start 142.125 94.375) (end 142.56 94.81) (width 0.2) (layer "F.Cu") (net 6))
 (segment (start 142.125 93.6) (end 142.125 94.375) (width 0.2) (layer "F.Cu") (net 6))
 (segment (start 146.05 91) (end 143.975 91) (width 0.2) (layer "F.Cu") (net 9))
 (segment (start 143.975 91) (end 143.85 90.875) (width 0.2) (layer "F.Cu") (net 9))
 (segment (start 143.8625 96.5) (end 144.45 96.5) (width 0.2) (layer "F.Cu") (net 1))
 (segment (start 144.45 96.5) (end 144.87 96.08) (width 0.2) (layer "F.Cu") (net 1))
 (segment (start 144.87 96.08) (end 146.05 96.08) (width 0.2) (layer "F.Cu") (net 1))
 (segment (start 133.96 97.5) (end 133.96 87.64) (width 0.2) (layer "F.Cu") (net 17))
 (segment (start 133.96 87.64) (end 134.65 86.95) (width 0.2) (layer "F.Cu") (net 17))
 (via (at 134.65 86.95) (size 0.6) (drill 0.3) (layers "F.Cu" "B.Cu") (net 17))
 (segment (start 134.65 86.95) (end 144.355 86.95) (width 0.2) (layer "B.Cu") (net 17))
 (segment (start 144.355 86.95) (end 145.565 85.74) (width 0.2) (layer "B.Cu") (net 17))
 (segment (start 149.15 91.394999) (end 150.025001 92.27) (width 0.2) (layer "F.Cu") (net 15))
 (segment (start 150.025001 92.27) (end 151 92.27) (width 0.2) (layer "F.Cu") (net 15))
 (segment (start 149.15 87.65) (end 149.15 91.394999) (width 0.2) (layer "F.Cu") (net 15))
 (segment (start 143.275 85.74) (end 144.735 87.2) (width 0.2) (layer "F.Cu") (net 15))
 (segment (start 148.7 87.2) (end 149.15 87.65) (width 0.2) (layer "F.Cu") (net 15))
 (segment (start 144.735 87.2) (end 148.7 87.2) (width 0.2) (layer "F.Cu") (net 15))
 (segment (start 142.846 87.601) (end 140.985 85.74) (width 0.2) (layer "F.Cu") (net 14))
 (segment (start 150.09 93.54) (end 148.749 92.199) (width 0.2) (layer "F.Cu") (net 14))
 (segment (start 148.5339 87.601) (end 142.846 87.601) (width 0.2) (layer "F.Cu") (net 14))
 (segment (start 148.749 92.199) (end 148.749 87.8161) (width 0.2) (layer "F.Cu") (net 14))
 (segment (start 151 93.54) (end 150.09 93.54) (width 0.2) (layer "F.Cu") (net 14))
 (segment (start 148.749 87.8161) (end 148.5339 87.601) (width 0.2) (layer "F.Cu") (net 14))
 (segment (start 151 94.81) (end 156.31 94.81) (width 0.2) (layer "F.Cu") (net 8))
 (segment (start 156.31 94.81) (end 156.96 95.46) (width 0.2) (layer "F.Cu") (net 8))
 (segment (start 156.96 95.46) (end 156.96 97.5) (width 0.2) (layer "F.Cu") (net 8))
 (segment (start 151.974999 96.08) (end 152.600331 96.705332) (width 0.2) (layer "F.Cu") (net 7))
 (segment (start 158.895369 98.890125) (end 158.900239 98.894995) (width 0.2) (layer "F.Cu") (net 7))
 (segment (start 155.740125 98.890125) (end 158.895369 98.890125) (width 0.2) (layer "F.Cu") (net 7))
 (segment (start 159.5 98.295234) (end 159.5 97.5) (width 0.2) (layer "F.Cu") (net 7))
 (segment (start 152.600331 96.705332) (end 152.600331 98.885287) (width 0.2) (layer "F.Cu") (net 7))
 (segment (start 152.600331 98.885287) (end 155.740125 98.890125) (width 0.2) (layer "F.Cu") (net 7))
 (segment (start 151 96.08) (end 151.974999 96.08) (width 0.2) (layer "F.Cu") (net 7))
 (segment (start 158.900239 98.894995) (end 159.5 98.295234) (width 0.2) (layer "F.Cu") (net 7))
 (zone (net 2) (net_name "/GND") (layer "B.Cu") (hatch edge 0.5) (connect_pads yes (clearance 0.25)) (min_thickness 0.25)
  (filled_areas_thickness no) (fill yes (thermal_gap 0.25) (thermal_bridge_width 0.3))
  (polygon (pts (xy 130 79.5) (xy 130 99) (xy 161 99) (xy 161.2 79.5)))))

